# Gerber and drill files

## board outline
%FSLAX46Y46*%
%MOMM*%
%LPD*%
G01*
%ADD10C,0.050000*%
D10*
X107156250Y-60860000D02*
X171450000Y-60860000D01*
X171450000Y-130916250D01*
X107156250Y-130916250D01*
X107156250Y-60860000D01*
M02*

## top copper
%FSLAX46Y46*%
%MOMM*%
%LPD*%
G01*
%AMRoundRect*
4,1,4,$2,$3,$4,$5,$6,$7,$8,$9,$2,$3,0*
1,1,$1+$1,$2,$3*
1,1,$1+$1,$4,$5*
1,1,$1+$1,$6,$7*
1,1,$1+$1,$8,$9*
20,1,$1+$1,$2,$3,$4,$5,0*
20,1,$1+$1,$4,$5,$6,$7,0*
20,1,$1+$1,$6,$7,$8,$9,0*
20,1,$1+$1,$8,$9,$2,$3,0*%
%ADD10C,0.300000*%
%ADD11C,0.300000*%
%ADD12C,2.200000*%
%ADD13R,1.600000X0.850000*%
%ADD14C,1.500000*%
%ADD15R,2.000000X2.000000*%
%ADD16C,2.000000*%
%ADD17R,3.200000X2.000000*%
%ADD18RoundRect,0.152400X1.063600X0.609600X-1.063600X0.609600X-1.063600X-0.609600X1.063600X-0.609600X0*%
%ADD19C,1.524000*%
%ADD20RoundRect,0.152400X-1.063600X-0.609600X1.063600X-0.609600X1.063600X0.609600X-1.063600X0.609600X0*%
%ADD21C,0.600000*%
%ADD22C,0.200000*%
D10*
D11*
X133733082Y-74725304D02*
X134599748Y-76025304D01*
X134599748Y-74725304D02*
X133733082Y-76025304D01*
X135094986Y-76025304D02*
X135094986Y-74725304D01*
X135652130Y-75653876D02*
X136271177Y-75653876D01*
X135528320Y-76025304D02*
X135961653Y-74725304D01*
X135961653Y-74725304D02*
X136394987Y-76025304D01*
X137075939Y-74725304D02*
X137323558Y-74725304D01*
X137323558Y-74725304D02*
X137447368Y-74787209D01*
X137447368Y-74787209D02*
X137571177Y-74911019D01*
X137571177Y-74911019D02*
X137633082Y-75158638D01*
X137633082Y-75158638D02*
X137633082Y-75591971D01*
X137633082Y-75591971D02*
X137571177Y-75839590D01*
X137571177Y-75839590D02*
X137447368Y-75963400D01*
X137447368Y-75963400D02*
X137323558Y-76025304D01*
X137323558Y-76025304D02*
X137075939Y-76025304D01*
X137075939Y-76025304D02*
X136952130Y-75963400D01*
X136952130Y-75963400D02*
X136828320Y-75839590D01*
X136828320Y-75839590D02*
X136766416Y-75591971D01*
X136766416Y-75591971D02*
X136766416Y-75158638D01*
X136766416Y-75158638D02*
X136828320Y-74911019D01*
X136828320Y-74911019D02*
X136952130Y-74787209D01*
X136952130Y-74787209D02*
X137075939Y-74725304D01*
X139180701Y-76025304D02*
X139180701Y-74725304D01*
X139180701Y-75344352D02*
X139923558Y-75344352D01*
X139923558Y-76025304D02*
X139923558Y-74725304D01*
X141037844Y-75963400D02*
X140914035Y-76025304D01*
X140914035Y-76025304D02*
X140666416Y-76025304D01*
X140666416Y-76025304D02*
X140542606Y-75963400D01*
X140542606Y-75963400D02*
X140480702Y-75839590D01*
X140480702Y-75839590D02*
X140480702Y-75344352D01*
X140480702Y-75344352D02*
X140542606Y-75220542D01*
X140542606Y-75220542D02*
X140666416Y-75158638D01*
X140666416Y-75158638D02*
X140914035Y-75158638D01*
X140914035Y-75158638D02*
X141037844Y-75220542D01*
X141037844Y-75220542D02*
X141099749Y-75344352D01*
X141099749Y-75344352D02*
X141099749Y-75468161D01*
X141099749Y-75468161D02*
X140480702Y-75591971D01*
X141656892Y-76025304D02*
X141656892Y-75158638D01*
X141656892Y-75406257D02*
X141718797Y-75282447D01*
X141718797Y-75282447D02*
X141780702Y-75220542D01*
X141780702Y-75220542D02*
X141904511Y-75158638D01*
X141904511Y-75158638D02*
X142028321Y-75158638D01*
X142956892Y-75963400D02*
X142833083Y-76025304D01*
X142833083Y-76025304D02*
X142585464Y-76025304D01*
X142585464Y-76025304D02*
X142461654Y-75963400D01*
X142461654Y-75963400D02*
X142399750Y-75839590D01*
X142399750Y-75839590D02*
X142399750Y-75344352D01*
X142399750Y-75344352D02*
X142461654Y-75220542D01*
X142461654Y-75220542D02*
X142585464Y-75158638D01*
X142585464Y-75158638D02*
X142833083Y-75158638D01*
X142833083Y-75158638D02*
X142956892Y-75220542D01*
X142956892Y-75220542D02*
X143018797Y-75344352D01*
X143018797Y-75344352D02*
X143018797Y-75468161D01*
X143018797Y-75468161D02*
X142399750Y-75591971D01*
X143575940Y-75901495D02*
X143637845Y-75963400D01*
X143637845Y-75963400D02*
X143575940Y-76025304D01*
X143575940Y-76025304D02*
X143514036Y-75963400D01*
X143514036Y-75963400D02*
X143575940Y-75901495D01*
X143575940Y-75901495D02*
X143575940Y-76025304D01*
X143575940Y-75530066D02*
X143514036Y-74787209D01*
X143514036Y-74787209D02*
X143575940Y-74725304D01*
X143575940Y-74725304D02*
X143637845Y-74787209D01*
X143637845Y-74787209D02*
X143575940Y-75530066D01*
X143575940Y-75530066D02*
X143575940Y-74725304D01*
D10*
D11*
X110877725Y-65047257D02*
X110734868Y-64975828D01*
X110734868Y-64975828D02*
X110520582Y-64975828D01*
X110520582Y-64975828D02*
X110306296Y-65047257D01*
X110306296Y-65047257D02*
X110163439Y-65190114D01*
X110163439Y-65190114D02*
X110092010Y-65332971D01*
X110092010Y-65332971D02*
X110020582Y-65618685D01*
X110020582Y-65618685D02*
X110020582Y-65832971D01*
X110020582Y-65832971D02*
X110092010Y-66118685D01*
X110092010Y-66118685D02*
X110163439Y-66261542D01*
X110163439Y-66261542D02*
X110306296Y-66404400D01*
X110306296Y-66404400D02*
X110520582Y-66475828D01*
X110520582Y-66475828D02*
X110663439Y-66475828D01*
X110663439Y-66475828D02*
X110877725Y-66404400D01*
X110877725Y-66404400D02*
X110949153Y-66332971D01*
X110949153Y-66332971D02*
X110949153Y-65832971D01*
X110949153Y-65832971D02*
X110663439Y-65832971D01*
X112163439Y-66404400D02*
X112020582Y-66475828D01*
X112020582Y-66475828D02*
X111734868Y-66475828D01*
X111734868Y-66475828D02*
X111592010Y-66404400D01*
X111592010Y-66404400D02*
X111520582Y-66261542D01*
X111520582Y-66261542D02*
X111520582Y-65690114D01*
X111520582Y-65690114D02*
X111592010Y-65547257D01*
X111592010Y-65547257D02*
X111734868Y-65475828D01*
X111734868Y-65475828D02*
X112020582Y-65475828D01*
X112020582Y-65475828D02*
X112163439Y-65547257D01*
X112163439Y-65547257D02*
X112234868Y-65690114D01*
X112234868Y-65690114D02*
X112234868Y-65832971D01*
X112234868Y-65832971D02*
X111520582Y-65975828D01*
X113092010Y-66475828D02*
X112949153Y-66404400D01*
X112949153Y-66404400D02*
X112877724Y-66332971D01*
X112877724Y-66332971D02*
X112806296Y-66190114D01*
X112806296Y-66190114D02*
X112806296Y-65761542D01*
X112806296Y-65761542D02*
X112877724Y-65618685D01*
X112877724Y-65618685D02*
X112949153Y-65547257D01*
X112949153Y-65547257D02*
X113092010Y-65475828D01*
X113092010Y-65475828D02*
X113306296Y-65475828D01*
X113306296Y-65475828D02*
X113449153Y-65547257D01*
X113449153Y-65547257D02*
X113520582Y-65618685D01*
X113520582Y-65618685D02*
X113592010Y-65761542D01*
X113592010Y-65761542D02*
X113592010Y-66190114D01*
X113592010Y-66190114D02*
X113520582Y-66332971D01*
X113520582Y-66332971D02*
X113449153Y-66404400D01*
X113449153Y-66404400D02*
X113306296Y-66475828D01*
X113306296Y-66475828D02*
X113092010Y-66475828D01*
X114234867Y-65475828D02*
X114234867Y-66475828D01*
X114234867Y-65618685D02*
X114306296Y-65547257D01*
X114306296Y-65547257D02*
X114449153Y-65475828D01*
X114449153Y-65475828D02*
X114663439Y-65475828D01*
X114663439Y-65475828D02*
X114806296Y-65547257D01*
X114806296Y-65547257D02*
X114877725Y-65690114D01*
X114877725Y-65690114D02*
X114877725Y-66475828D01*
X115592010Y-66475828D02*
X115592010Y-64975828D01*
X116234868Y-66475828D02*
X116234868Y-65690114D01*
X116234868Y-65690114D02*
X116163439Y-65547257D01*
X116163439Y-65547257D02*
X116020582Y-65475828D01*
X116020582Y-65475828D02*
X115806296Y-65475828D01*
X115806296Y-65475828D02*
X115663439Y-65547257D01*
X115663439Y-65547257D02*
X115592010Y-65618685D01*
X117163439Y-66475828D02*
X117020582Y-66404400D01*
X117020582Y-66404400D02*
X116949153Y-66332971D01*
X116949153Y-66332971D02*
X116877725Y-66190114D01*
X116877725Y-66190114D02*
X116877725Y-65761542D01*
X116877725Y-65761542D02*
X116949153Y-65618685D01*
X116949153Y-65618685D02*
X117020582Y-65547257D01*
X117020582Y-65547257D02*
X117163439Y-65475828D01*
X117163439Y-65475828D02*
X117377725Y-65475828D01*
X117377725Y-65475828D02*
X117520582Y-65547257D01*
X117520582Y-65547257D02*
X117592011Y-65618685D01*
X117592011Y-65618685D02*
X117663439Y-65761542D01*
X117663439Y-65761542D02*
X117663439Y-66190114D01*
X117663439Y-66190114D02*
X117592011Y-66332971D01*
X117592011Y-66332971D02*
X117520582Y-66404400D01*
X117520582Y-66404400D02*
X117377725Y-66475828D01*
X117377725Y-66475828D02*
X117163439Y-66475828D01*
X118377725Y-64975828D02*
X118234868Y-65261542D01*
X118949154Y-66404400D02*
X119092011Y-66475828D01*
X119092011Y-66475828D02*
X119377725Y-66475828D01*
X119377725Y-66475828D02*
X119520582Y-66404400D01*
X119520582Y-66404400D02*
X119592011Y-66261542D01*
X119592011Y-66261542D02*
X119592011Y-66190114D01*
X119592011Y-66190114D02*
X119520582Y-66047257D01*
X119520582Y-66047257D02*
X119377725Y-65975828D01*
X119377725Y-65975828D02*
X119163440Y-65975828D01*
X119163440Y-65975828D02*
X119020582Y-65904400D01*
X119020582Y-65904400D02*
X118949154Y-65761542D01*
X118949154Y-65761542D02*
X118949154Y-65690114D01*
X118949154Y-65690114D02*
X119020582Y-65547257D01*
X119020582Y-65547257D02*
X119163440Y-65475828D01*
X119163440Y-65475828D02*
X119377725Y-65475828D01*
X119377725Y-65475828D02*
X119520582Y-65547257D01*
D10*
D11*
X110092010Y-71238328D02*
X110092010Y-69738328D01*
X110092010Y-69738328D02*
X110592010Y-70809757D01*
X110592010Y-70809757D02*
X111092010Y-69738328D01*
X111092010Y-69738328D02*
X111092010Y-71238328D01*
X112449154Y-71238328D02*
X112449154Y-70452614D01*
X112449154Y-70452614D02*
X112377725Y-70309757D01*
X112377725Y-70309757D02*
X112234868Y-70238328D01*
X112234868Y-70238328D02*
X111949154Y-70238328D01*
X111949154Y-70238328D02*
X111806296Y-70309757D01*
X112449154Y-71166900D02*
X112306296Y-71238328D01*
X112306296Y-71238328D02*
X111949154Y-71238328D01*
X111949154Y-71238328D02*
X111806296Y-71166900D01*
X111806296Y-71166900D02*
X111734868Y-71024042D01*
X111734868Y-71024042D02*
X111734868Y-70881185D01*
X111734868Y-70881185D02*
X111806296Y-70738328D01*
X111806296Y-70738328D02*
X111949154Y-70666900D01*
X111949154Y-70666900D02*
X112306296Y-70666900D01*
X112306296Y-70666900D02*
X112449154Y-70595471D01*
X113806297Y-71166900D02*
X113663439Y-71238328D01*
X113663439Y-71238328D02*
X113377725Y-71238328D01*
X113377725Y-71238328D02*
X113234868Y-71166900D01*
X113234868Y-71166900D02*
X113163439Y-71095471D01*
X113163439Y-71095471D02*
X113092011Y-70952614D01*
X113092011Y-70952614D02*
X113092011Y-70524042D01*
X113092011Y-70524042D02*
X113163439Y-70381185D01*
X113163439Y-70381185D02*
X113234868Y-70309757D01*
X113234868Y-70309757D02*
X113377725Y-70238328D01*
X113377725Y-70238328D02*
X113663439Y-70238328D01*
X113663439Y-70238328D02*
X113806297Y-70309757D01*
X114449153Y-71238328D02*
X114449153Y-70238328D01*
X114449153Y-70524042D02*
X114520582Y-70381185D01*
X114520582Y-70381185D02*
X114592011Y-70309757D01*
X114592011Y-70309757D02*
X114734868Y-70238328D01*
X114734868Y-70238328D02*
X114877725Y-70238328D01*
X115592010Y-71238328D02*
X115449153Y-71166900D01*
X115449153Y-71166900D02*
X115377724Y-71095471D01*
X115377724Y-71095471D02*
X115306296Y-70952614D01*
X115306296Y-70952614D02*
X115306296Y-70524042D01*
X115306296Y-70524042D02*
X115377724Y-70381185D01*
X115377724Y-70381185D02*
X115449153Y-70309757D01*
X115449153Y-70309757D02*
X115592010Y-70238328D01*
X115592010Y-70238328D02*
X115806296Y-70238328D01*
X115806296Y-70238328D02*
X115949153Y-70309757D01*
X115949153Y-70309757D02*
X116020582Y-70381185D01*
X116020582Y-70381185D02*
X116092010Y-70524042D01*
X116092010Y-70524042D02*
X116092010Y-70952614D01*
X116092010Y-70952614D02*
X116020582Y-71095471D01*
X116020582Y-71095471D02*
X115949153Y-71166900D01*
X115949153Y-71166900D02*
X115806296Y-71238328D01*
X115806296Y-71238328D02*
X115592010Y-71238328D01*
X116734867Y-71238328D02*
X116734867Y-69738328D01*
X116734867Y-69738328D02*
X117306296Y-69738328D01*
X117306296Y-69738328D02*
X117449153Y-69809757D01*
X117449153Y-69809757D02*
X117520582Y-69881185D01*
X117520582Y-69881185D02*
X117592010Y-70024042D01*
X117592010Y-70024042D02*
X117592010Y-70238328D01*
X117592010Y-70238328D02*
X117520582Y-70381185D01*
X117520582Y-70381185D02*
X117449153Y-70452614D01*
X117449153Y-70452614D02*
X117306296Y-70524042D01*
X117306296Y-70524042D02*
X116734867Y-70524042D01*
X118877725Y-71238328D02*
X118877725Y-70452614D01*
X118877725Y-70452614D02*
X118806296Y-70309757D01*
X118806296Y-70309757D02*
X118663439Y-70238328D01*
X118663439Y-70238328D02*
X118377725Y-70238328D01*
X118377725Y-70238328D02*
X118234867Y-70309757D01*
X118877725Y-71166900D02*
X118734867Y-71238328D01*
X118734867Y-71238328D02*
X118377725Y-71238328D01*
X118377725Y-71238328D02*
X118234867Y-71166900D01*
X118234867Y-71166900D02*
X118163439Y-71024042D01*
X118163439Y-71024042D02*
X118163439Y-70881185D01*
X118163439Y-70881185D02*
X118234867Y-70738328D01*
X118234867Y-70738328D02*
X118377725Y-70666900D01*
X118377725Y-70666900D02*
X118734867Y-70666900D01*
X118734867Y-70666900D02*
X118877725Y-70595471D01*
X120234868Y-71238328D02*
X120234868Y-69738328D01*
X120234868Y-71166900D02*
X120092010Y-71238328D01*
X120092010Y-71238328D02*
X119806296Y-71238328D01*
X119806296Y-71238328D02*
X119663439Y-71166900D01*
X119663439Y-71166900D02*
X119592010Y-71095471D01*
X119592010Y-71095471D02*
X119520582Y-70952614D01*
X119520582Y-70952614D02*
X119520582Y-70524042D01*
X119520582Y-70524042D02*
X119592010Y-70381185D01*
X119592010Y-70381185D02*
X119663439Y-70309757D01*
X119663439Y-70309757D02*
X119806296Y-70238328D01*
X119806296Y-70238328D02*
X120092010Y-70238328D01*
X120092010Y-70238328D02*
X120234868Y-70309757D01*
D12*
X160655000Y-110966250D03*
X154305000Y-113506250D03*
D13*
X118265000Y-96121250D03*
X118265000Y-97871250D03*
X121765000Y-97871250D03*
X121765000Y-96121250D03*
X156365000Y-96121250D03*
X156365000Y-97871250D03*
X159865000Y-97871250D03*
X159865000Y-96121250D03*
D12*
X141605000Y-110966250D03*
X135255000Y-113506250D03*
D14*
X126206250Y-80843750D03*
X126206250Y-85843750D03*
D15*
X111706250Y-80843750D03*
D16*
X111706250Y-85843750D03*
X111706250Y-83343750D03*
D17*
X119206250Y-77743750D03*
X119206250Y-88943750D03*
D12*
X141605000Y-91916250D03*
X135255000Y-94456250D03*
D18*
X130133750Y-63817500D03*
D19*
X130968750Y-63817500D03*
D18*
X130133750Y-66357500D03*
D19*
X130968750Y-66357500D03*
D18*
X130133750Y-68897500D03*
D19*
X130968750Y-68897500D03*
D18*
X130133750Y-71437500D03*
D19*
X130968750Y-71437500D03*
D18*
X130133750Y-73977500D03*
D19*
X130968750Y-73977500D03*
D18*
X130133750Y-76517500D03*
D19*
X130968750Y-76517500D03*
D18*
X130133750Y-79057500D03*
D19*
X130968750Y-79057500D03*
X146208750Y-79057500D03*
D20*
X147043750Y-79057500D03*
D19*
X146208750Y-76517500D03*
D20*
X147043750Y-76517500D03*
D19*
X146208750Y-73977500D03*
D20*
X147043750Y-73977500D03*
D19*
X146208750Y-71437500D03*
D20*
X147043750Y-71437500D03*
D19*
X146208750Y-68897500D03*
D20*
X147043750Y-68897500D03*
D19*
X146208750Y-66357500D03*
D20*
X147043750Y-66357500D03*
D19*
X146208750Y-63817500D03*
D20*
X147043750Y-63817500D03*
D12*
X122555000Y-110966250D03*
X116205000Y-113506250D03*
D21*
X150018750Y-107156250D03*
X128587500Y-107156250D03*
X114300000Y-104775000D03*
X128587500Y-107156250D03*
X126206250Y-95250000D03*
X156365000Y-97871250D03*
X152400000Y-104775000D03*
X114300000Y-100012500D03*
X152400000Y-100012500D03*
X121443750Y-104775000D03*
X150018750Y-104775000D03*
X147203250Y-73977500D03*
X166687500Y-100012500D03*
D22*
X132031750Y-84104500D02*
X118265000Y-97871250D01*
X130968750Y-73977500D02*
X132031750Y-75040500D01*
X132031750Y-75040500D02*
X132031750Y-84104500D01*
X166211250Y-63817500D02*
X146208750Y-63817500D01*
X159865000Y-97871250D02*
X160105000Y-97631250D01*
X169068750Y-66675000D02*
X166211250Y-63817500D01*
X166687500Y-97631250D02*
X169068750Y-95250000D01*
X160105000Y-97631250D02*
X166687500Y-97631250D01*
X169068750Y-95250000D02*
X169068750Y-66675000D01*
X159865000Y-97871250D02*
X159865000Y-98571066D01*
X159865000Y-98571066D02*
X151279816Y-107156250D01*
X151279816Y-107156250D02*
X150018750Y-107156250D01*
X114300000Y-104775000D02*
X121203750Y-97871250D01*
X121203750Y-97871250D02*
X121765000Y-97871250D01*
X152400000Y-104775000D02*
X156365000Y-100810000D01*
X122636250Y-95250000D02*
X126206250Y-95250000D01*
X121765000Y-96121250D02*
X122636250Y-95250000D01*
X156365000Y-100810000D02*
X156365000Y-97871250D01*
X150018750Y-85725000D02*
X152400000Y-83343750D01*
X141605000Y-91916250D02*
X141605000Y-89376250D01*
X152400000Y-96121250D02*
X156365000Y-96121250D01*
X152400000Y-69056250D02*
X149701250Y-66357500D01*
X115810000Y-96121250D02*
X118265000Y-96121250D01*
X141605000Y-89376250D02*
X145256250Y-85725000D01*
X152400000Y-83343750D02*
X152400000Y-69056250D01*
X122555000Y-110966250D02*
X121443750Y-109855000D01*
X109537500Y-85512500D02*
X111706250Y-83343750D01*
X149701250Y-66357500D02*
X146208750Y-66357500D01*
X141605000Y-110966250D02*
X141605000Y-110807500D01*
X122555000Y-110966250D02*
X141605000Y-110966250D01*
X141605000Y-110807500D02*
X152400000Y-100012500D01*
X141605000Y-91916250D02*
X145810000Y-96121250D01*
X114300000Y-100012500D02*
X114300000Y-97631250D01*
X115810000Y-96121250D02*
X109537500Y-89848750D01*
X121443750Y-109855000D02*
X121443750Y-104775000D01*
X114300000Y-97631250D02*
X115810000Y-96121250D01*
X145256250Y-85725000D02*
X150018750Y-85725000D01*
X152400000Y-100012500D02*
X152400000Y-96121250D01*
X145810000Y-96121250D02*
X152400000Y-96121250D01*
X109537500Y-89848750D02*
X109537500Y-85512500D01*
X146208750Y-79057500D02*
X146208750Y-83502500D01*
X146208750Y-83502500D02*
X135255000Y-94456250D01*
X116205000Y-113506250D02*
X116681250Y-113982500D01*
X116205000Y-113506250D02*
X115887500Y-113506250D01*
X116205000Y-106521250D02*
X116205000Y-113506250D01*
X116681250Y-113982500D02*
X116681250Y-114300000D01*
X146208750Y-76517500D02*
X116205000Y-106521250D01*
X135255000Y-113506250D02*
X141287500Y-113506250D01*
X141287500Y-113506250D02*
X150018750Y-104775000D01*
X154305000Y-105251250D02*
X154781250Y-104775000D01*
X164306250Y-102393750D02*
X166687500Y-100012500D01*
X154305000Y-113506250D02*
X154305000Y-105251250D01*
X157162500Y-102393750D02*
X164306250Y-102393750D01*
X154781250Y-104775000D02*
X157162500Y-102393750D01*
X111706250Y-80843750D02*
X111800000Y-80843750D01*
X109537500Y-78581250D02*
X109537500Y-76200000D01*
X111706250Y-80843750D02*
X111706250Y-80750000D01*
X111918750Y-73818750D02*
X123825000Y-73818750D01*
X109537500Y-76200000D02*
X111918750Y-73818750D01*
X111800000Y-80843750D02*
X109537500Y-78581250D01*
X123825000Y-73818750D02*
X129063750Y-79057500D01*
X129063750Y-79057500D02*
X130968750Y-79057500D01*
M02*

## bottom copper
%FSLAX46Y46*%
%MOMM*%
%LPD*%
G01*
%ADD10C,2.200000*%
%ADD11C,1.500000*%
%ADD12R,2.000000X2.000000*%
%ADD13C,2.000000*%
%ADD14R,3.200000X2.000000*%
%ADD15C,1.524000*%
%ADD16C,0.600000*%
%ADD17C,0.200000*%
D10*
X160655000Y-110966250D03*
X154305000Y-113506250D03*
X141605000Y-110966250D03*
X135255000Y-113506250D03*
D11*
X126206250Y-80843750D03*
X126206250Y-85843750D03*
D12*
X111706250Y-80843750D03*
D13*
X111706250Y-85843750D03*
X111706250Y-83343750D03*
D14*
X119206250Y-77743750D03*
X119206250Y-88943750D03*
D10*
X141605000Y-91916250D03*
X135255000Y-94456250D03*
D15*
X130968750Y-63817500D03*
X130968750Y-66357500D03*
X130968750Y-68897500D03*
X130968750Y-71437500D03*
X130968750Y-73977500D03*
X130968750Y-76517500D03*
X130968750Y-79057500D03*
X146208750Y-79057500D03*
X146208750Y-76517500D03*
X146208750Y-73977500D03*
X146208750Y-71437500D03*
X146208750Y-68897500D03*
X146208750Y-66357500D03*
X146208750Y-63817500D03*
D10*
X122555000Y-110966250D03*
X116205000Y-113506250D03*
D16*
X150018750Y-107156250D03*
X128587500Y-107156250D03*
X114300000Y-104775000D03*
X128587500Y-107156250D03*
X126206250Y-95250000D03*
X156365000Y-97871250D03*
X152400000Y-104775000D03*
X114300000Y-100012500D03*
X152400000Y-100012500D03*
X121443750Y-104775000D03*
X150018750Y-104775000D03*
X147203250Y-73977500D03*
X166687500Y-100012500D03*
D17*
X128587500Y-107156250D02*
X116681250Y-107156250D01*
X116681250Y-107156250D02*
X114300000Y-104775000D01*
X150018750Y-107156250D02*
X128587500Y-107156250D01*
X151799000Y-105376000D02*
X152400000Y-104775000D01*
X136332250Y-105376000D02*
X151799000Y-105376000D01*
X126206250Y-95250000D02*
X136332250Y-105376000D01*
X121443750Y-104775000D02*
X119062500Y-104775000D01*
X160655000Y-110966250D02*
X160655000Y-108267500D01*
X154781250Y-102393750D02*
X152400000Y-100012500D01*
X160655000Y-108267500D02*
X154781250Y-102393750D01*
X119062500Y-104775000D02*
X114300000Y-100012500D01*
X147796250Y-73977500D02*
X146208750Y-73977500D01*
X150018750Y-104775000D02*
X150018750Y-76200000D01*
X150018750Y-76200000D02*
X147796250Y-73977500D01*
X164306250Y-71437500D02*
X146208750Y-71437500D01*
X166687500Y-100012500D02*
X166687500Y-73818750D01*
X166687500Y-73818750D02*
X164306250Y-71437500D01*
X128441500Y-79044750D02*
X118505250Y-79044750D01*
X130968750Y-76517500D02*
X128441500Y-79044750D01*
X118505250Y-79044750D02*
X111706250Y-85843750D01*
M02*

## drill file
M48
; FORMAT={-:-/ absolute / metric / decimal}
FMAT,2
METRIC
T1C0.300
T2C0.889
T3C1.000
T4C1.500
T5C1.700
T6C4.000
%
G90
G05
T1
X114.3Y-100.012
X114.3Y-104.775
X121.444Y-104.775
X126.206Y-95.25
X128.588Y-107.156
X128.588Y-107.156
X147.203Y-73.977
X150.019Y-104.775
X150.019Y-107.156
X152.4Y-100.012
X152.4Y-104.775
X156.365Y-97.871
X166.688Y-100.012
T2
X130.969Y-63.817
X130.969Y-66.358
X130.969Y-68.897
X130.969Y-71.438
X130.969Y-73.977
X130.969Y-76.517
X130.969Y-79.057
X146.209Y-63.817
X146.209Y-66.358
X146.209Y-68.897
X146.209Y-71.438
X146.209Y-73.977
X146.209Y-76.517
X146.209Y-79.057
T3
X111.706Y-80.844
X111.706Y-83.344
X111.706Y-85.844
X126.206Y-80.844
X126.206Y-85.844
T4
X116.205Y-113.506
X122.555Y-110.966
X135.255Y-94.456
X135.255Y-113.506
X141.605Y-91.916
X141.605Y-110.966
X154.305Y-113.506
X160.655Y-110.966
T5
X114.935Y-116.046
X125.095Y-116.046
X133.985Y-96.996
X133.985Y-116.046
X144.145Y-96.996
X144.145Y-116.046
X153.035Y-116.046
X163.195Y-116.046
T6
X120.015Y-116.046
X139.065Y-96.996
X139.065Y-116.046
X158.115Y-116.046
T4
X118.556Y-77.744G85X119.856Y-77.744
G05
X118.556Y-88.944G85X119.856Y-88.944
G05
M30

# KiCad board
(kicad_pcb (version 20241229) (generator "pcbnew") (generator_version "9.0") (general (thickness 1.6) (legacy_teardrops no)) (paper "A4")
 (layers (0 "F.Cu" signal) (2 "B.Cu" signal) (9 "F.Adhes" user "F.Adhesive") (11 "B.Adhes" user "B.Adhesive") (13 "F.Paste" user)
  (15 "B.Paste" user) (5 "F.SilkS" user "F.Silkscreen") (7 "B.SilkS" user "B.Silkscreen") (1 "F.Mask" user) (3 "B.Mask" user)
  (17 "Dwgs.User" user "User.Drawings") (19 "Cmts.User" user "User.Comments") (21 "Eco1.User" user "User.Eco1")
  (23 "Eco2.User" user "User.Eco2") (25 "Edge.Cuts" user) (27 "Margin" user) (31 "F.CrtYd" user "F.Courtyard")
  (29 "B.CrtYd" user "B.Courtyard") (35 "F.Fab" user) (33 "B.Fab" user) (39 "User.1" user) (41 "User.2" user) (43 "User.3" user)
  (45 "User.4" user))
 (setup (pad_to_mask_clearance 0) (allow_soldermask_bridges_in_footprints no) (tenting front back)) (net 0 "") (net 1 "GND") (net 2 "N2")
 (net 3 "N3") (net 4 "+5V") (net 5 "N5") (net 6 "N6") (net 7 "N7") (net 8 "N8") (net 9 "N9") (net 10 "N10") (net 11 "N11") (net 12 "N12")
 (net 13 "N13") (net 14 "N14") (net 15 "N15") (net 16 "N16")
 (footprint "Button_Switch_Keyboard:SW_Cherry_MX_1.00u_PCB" (layer "F.Cu") (at 160.655 110.96625)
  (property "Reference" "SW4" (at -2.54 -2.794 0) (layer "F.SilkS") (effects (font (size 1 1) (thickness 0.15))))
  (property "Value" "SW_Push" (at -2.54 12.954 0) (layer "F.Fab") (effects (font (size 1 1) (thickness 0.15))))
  (pad "" np_thru_hole circle (at -7.62 5.08) (size 1.7 1.7) (drill 1.7) (layers "*.Cu" "*.Mask"))
  (pad "" np_thru_hole circle (at -2.54 5.08) (size 4 4) (drill 4) (layers "*.Cu" "*.Mask"))
  (pad "" np_thru_hole circle (at 2.54 5.08) (size 1.7 1.7) (drill 1.7) (layers "*.Cu" "*.Mask"))
  (pad "1" thru_hole circle (at 0 0) (size 2.2 2.2) (drill 1.5) (layers "*.Cu" "*.Mask") (remove_unused_layers no) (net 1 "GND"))
  (pad "2" thru_hole circle (at -6.35 2.54) (size 2.2 2.2) (drill 1.5) (layers "*.Cu" "*.Mask") (remove_unused_layers no) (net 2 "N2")))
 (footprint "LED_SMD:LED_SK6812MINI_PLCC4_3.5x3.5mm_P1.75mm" (layer "F.Cu") (at 120.015 96.99625)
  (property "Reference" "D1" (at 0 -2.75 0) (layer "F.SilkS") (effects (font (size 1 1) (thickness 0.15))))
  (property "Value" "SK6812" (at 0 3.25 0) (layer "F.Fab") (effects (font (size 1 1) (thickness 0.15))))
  (pad "1" smd rect (at -1.75 -0.875) (size 1.6 0.85) (layers "F.Cu" "F.Mask" "F.Paste") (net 1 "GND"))
  (pad "2" smd rect (at -1.75 0.875) (size 1.6 0.85) (layers "F.Cu" "F.Mask" "F.Paste") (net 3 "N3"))
  (pad "3" smd rect (at 1.75 0.875) (size 1.6 0.85) (layers "F.Cu" "F.Mask" "F.Paste") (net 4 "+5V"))
  (pad "4" smd rect (at 1.75 -0.875) (size 1.6 0.85) (layers "F.Cu" "F.Mask" "F.Paste") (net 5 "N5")))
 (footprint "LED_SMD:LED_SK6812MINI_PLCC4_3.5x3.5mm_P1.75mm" (layer "F.Cu") (at 158.115 96.99625)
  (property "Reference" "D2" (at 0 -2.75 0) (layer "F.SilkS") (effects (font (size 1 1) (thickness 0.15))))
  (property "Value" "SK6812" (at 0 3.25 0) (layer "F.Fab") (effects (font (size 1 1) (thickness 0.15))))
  (pad "1" smd rect (at -1.75 -0.875) (size 1.6 0.85) (layers "F.Cu" "F.Mask" "F.Paste") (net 1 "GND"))
  (pad "2" smd rect (at -1.75 0.875) (size 1.6 0.85) (layers "F.Cu" "F.Mask" "F.Paste") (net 5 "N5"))
  (pad "3" smd rect (at 1.75 0.875) (size 1.6 0.85) (layers "F.Cu" "F.Mask" "F.Paste") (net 4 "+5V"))
  (pad "4" smd rect (at 1.75 -0.875) (size 1.6 0.85) (layers "F.Cu" "F.Mask" "F.Paste") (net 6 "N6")))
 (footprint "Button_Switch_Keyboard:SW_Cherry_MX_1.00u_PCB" (layer "F.Cu") (at 141.605 110.96625)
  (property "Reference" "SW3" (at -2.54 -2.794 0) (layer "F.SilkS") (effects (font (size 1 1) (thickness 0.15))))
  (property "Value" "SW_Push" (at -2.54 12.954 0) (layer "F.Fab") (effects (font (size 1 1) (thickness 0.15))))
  (pad "" np_thru_hole circle (at -7.62 5.08) (size 1.7 1.7) (drill 1.7) (layers "*.Cu" "*.Mask"))
  (pad "" np_thru_hole circle (at -2.54 5.08) (size 4 4) (drill 4) (layers "*.Cu" "*.Mask"))
  (pad "" np_thru_hole circle (at 2.54 5.08) (size 1.7 1.7) (drill 1.7) (layers "*.Cu" "*.Mask"))
  (pad "1" thru_hole circle (at 0 0) (size 2.2 2.2) (drill 1.5) (layers "*.Cu" "*.Mask") (remove_unused_layers no) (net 1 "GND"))
  (pad "2" thru_hole circle (at -6.35 2.54) (size 2.2 2.2) (drill 1.5) (layers "*.Cu" "*.Mask") (remove_unused_layers no) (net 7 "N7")))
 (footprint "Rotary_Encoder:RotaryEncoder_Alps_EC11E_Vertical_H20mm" (layer "F.Cu") (at 111.70625 80.84375)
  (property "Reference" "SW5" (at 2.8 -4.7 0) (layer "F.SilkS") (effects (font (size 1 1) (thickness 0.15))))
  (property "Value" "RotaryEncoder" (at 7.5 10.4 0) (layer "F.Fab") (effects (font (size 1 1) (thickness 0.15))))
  (pad "" thru_hole circle (at 14.5 0) (size 1.5 1.5) (drill 1) (layers "*.Cu" "*.Mask") (remove_unused_layers no))
  (pad "" thru_hole circle (at 14.5 5) (size 1.5 1.5) (drill 1) (layers "*.Cu" "*.Mask") (remove_unused_layers no))
  (pad "A" thru_hole rect (at 0 0) (size 2 2) (drill 1) (layers "*.Cu" "*.Mask") (remove_unused_layers no) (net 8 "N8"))
  (pad "B" thru_hole circle (at 0 5) (size 2 2) (drill 1) (layers "*.Cu" "*.Mask") (remove_unused_layers no) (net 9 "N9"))
  (pad "C" thru_hole circle (at 0 2.5) (size 2 2) (drill 1) (layers "*.Cu" "*.Mask") (remove_unused_layers no) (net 1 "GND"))
  (pad "MP" thru_hole rect (at 7.5 -3.1) (size 3.2 2) (drill oval 2.8 1.5) (layers "*.Cu" "*.Mask") (remove_unused_layers no))
  (pad "MP" thru_hole rect (at 7.5 8.1) (size 3.2 2) (drill oval 2.8 1.5) (layers "*.Cu" "*.Mask") (remove_unused_layers no)))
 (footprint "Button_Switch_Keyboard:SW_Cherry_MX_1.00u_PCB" (layer "F.Cu") (at 141.605 91.91625)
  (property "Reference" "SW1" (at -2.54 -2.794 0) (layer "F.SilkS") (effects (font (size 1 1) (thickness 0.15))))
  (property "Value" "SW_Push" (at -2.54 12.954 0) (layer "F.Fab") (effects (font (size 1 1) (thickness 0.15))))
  (pad "" np_thru_hole circle (at -7.62 5.08) (size 1.7 1.7) (drill 1.7) (layers "*.Cu" "*.Mask"))
  (pad "" np_thru_hole circle (at -2.54 5.08) (size 4 4) (drill 4) (layers "*.Cu" "*.Mask"))
  (pad "" np_thru_hole circle (at 2.54 5.08) (size 1.7 1.7) (drill 1.7) (layers "*.Cu" "*.Mask"))
  (pad "1" thru_hole circle (at 0 0) (size 2.2 2.2) (drill 1.5) (layers "*.Cu" "*.Mask") (remove_unused_layers no) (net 1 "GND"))
  (pad "2" thru_hole circle (at -6.35 2.54) (size 2.2 2.2) (drill 1.5) (layers "*.Cu" "*.Mask") (remove_unused_layers no) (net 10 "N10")))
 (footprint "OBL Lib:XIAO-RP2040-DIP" (layer "F.Cu") (at 138.58875 71.4375)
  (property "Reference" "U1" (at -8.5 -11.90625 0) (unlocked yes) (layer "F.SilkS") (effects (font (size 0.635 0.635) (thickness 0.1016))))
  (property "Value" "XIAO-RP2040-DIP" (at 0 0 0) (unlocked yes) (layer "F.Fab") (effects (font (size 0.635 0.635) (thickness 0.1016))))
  (pad "1" smd roundrect (at -8.455 -7.62 180) (size 2.432 1.524) (layers "F.Cu" "F.Mask") (roundrect_rratio 0.1) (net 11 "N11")
   (thermal_bridge_angle 45))
  (pad "1" thru_hole circle (at -7.62 -7.62 180) (size 1.524 1.524) (drill 0.889) (layers "*.Cu" "*.Mask") (remove_unused_layers no)
   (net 11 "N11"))
  (pad "2" smd roundrect (at -8.455 -5.08 180) (size 2.432 1.524) (layers "F.Cu" "F.Mask") (roundrect_rratio 0.1) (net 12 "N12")
   (thermal_bridge_angle 45))
  (pad "2" thru_hole circle (at -7.62 -5.08 180) (size 1.524 1.524) (drill 0.889) (layers "*.Cu" "*.Mask") (remove_unused_layers no)
   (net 12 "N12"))
  (pad "3" smd roundrect (at -8.455 -2.54 180) (size 2.432 1.524) (layers "F.Cu" "F.Mask") (roundrect_rratio 0.1) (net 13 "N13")
   (thermal_bridge_angle 45))
  (pad "3" thru_hole circle (at -7.62 -2.54 180) (size 1.524 1.524) (drill 0.889) (layers "*.Cu" "*.Mask") (remove_unused_layers no)
   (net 13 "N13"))
  (pad "4" smd roundrect (at -8.455 0 180) (size 2.432 1.524) (layers "F.Cu" "F.Mask") (roundrect_rratio 0.1) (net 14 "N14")
   (thermal_bridge_angle 45))
  (pad "4" thru_hole circle (at -7.62 0 180) (size 1.524 1.524) (drill 0.889) (layers "*.Cu" "*.Mask") (remove_unused_layers no)
   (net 14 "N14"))
  (pad "5" smd roundrect (at -8.455 2.54 180) (size 2.432 1.524) (layers "F.Cu" "F.Mask") (roundrect_rratio 0.1) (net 3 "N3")
   (thermal_bridge_angle 45))
  (pad "5" thru_hole circle (at -7.62 2.54 180) (size 1.524 1.524) (drill 0.889) (layers "*.Cu" "*.Mask") (remove_unused_layers no)
   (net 3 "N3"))
  (pad "6" smd roundrect (at -8.455 5.08 180) (size 2.432 1.524) (layers "F.Cu" "F.Mask") (roundrect_rratio 0.1) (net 9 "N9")
   (thermal_bridge_angle 45))
  (pad "6" thru_hole circle (at -7.62 5.08 180) (size 1.524 1.524) (drill 0.889) (layers "*.Cu" "*.Mask") (remove_unused_layers no)
   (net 9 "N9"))
  (pad "7" smd roundrect (at -8.455 7.62 180) (size 2.432 1.524) (layers "F.Cu" "F.Mask") (roundrect_rratio 0.1) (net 8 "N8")
   (thermal_bridge_angle 45))
  (pad "7" thru_hole circle (at -7.62 7.62 180) (size 1.524 1.524) (drill 0.889) (layers "*.Cu" "*.Mask") (remove_unused_layers no)
   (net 8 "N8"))
  (pad "8" thru_hole circle (at 7.62 7.62) (size 1.524 1.524) (drill 0.889) (layers "*.Cu" "*.Mask") (remove_unused_layers no)
   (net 10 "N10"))
  (pad "8" smd roundrect (at 8.455 7.62) (size 2.432 1.524) (layers "F.Cu" "F.Mask") (roundrect_rratio 0.1) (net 10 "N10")
   (thermal_bridge_angle 45))
  (pad "9" thru_hole circle (at 7.62 5.08) (size 1.524 1.524) (drill 0.889) (layers "*.Cu" "*.Mask") (remove_unused_layers no)
   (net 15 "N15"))
  (pad "9" smd roundrect (at 8.455 5.08) (size 2.432 1.524) (layers "F.Cu" "F.Mask") (roundrect_rratio 0.1) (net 15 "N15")
   (thermal_bridge_angle 45))
  (pad "10" thru_hole circle (at 7.62 2.54) (size 1.524 1.524) (drill 0.889) (layers "*.Cu" "*.Mask") (remove_unused_layers no) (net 7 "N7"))
  (pad "10" smd roundrect (at 8.455 2.54) (size 2.432 1.524) (layers "F.Cu" "F.Mask") (roundrect_rratio 0.1) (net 7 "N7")
   (thermal_bridge_angle 45))
  (pad "11" thru_hole circle (at 7.62 0) (size 1.524 1.524) (drill 0.889) (layers "*.Cu" "*.Mask") (remove_unused_layers no) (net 2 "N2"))
  (pad "11" smd roundrect (at 8.455 0) (size 2.432 1.524) (layers "F.Cu" "F.Mask") (roundrect_rratio 0.1) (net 2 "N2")
   (thermal_bridge_angle 45))
  (pad "12" thru_hole circle (at 7.62 -2.54) (size 1.524 1.524) (drill 0.889) (layers "*.Cu" "*.Mask") (remove_unused_layers no)
   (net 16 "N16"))
  (pad "12" smd roundrect (at 8.455 -2.54) (size 2.432 1.524) (layers "F.Cu" "F.Mask") (roundrect_rratio 0.1) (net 16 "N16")
   (thermal_bridge_angle 45))
  (pad "13" thru_hole circle (at 7.62 -5.08) (size 1.524 1.524) (drill 0.889) (layers "*.Cu" "*.Mask") (remove_unused_layers no)
   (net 1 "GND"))
  (pad "13" smd roundrect (at 8.455 -5.08) (size 2.432 1.524) (layers "F.Cu" "F.Mask") (roundrect_rratio 0.1) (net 1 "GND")
   (thermal_bridge_angle 45))
  (pad "14" thru_hole circle (at 7.62 -7.62) (size 1.524 1.524) (drill 0.889) (layers "*.Cu" "*.Mask") (remove_unused_layers no)
   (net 4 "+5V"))
  (pad "14" smd roundrect (at 8.455 -7.62) (size 2.432 1.524) (layers "F.Cu" "F.Mask") (roundrect_rratio 0.1) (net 4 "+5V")
   (thermal_bridge_angle 45)))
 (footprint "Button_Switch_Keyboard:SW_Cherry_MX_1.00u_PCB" (layer "F.Cu") (at 122.555 110.96625)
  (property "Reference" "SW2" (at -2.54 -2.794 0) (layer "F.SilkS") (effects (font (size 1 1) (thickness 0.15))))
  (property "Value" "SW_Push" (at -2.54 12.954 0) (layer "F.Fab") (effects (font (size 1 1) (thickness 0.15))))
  (pad "" np_thru_hole circle (at -7.62 5.08) (size 1.7 1.7) (drill 1.7) (layers "*.Cu" "*.Mask"))
  (pad "" np_thru_hole circle (at -2.54 5.08) (size 4 4) (drill 4) (layers "*.Cu" "*.Mask"))
  (pad "" np_thru_hole circle (at 2.54 5.08) (size 1.7 1.7) (drill 1.7) (layers "*.Cu" "*.Mask"))
  (pad "1" thru_hole circle (at 0 0) (size 2.2 2.2) (drill 1.5) (layers "*.Cu" "*.Mask") (remove_unused_layers no) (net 1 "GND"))
  (pad "2" thru_hole circle (at -6.35 2.54) (size 2.2 2.2) (drill 1.5) (layers "*.Cu" "*.Mask") (remove_unused_layers no) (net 15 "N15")))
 (gr_rect (start 107.15625 60.86) (end 171.45 130.91625) (stroke (width 0.05) (type default)) (fill no) (layer "Edge.Cuts"))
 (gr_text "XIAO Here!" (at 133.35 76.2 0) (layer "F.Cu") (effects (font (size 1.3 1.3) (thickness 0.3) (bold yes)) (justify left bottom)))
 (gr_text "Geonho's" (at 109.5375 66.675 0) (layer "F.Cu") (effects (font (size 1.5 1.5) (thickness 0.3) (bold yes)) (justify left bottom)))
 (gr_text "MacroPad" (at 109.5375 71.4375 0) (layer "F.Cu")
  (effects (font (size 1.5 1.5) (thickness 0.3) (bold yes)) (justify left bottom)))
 (segment (start 132.03175 84.1045) (end 118.265 97.87125) (width 0.2) (layer "F.Cu") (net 3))
 (segment (start 130.96875 73.9775) (end 132.03175 75.0405) (width 0.2) (layer "F.Cu") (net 3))
 (segment (start 132.03175 75.0405) (end 132.03175 84.1045) (width 0.2) (layer "F.Cu") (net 3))
 (segment (start 166.21125 63.8175) (end 146.20875 63.8175) (width 0.2) (layer "F.Cu") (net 4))
 (segment (start 159.865 97.87125) (end 160.105 97.63125) (width 0.2) (layer "F.Cu") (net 4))
 (segment (start 169.06875 66.675) (end 166.21125 63.8175) (width 0.2) (layer "F.Cu") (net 4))
 (segment (start 166.6875 97.63125) (end 169.06875 95.25) (width 0.2) (layer "F.Cu") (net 4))
 (segment (start 160.105 97.63125) (end 166.6875 97.63125) (width 0.2) (layer "F.Cu") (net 4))
 (segment (start 169.06875 95.25) (end 169.06875 66.675) (width 0.2) (layer "F.Cu") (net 4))
 (segment (start 159.865 97.87125) (end 159.865 98.571066) (width 0.2) (layer "F.Cu") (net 4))
 (segment (start 159.865 98.571066) (end 151.279816 107.15625) (width 0.2) (layer "F.Cu") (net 4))
 (segment (start 151.279816 107.15625) (end 150.01875 107.15625) (width 0.2) (layer "F.Cu") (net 4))
 (segment (start 114.3 104.775) (end 121.20375 97.87125) (width 0.2) (layer "F.Cu") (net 4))
 (segment (start 121.20375 97.87125) (end 121.765 97.87125) (width 0.2) (layer "F.Cu") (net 4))
 (via (at 150.01875 107.15625) (size 0.6) (drill 0.3) (layers "F.Cu" "B.Cu") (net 4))
 (via (at 128.5875 107.15625) (size 0.6) (drill 0.3) (layers "F.Cu" "B.Cu") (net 4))
 (via (at 114.3 104.775) (size 0.6) (drill 0.3) (layers "F.Cu" "B.Cu") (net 4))
 (via (at 128.5875 107.15625) (size 0.6) (drill 0.3) (layers "F.Cu" "B.Cu") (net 4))
 (segment (start 128.5875 107.15625) (end 116.68125 107.15625) (width 0.2) (layer "B.Cu") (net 4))
 (segment (start 116.68125 107.15625) (end 114.3 104.775) (width 0.2) (layer "B.Cu") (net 4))
 (segment (start 150.01875 107.15625) (end 128.5875 107.15625) (width 0.2) (layer "B.Cu") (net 4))
 (segment (start 152.4 104.775) (end 156.365 100.81) (width 0.2) (layer "F.Cu") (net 5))
 (segment (start 122.63625 95.25) (end 126.20625 95.25) (width 0.2) (layer "F.Cu") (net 5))
 (segment (start 121.765 96.12125) (end 122.63625 95.25) (width 0.2) (layer "F.Cu") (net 5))
 (segment (start 156.365 100.81) (end 156.365 97.87125) (width 0.2) (layer "F.Cu") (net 5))
 (via (at 126.20625 95.25) (size 0.6) (drill 0.3) (layers "F.Cu" "B.Cu") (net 5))
 (via (at 156.365 97.87125) (size 0.6) (drill 0.3) (layers "F.Cu" "B.Cu") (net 5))
 (via (at 152.4 104.775) (size 0.6) (drill 0.3) (layers "F.Cu" "B.Cu") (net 5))
 (segment (start 151.799 105.376) (end 152.4 104.775) (width 0.2) (layer "B.Cu") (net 5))
 (segment (start 136.33225 105.376) (end 151.799 105.376) (width 0.2) (layer "B.Cu") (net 5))
 (segment (start 126.20625 95.25) (end 136.33225 105.376) (width 0.2) (layer "B.Cu") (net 5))
 (segment (start 150.01875 85.725) (end 152.4 83.34375) (width 0.2) (layer "F.Cu") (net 1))
 (segment (start 141.605 91.91625) (end 141.605 89.37625) (width 0.2) (layer "F.Cu") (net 1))
 (segment (start 152.4 96.12125) (end 156.365 96.12125) (width 0.2) (layer "F.Cu") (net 1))
 (segment (start 152.4 69.05625) (end 149.70125 66.3575) (width 0.2) (layer "F.Cu") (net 1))
 (segment (start 115.81 96.12125) (end 118.265 96.12125) (width 0.2) (layer "F.Cu") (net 1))
 (segment (start 141.605 89.37625) (end 145.25625 85.725) (width 0.2) (layer "F.Cu") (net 1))
 (segment (start 152.4 83.34375) (end 152.4 69.05625) (width 0.2) (layer "F.Cu") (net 1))
 (segment (start 122.555 110.96625) (end 121.44375 109.855) (width 0.2) (layer "F.Cu") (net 1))
 (segment (start 109.5375 85.5125) (end 111.70625 83.34375) (width 0.2) (layer "F.Cu") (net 1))
 (segment (start 149.70125 66.3575) (end 146.20875 66.3575) (width 0.2) (layer "F.Cu") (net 1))
 (segment (start 141.605 110.96625) (end 141.605 110.8075) (width 0.2) (layer "F.Cu") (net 1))
 (segment (start 122.555 110.96625) (end 141.605 110.96625) (width 0.2) (layer "F.Cu") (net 1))
 (segment (start 141.605 110.8075) (end 152.4 100.0125) (width 0.2) (layer "F.Cu") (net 1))
 (segment (start 141.605 91.91625) (end 145.81 96.12125) (width 0.2) (layer "F.Cu") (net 1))
 (segment (start 114.3 100.0125) (end 114.3 97.63125) (width 0.2) (layer "F.Cu") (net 1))
 (segment (start 115.81 96.12125) (end 109.5375 89.84875) (width 0.2) (layer "F.Cu") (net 1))
 (segment (start 121.44375 109.855) (end 121.44375 104.775) (width 0.2) (layer "F.Cu") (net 1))
 (segment (start 114.3 97.63125) (end 115.81 96.12125) (width 0.2) (layer "F.Cu") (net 1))
 (segment (start 145.25625 85.725) (end 150.01875 85.725) (width 0.2) (layer "F.Cu") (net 1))
 (segment (start 152.4 100.0125) (end 152.4 96.12125) (width 0.2) (layer "F.Cu") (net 1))
 (segment (start 145.81 96.12125) (end 152.4 96.12125) (width 0.2) (layer "F.Cu") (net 1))
 (segment (start 109.5375 89.84875) (end 109.5375 85.5125) (width 0.2) (layer "F.Cu") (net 1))
 (via (at 114.3 100.0125) (size 0.6) (drill 0.3) (layers "F.Cu" "B.Cu") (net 1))
 (via (at 152.4 100.0125) (size 0.6) (drill 0.3) (layers "F.Cu" "B.Cu") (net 1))
 (via (at 121.44375 104.775) (size 0.6) (drill 0.3) (layers "F.Cu" "B.Cu") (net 1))
 (segment (start 121.44375 104.775) (end 119.0625 104.775) (width 0.2) (layer "B.Cu") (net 1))
 (segment (start 160.655 110.96625) (end 160.655 108.2675) (width 0.2) (layer "B.Cu") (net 1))
 (segment (start 154.78125 102.39375) (end 152.4 100.0125) (width 0.2) (layer "B.Cu") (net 1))
 (segment (start 160.655 108.2675) (end 154.78125 102.39375) (width 0.2) (layer "B.Cu") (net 1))
 (segment (start 119.0625 104.775) (end 114.3 100.0125) (width 0.2) (layer "B.Cu") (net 1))
 (segment (start 146.20875 79.0575) (end 146.20875 83.5025) (width 0.2) (layer "F.Cu") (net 10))
 (segment (start 146.20875 83.5025) (end 135.255 94.45625) (width 0.2) (layer "F.Cu") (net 10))
 (segment (start 116.205 113.50625) (end 116.68125 113.9825) (width 0.2) (layer "F.Cu") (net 15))
 (segment (start 116.205 113.50625) (end 115.8875 113.50625) (width 0.2) (layer "F.Cu") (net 15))
 (segment (start 116.205 106.52125) (end 116.205 113.50625) (width 0.2) (layer "F.Cu") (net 15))
 (segment (start 116.68125 113.9825) (end 116.68125 114.3) (width 0.2) (layer "F.Cu") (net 15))
 (segment (start 146.20875 76.5175) (end 116.205 106.52125) (width 0.2) (layer "F.Cu") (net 15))
 (segment (start 135.255 113.50625) (end 141.2875 113.50625) (width 0.2) (layer "F.Cu") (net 7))
 (segment (start 141.2875 113.50625) (end 150.01875 104.775) (width 0.2) (layer "F.Cu") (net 7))
 (via (at 150.01875 104.775) (size 0.6) (drill 0.3) (layers "F.Cu" "B.Cu") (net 7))
 (via (at 147.20325 73.9775) (size 0.6) (drill 0.3) (layers "F.Cu" "B.Cu") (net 7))
 (segment (start 147.79625 73.9775) (end 146.20875 73.9775) (width 0.2) (layer "B.Cu") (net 7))
 (segment (start 150.01875 104.775) (end 150.01875 76.2) (width 0.2) (layer "B.Cu") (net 7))
 (segment (start 150.01875 76.2) (end 147.79625 73.9775) (width 0.2) (layer "B.Cu") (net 7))
 (segment (start 154.305 105.25125) (end 154.78125 104.775) (width 0.2) (layer "F.Cu") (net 2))
 (segment (start 164.30625 102.39375) (end 166.6875 100.0125) (width 0.2) (layer "F.Cu") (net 2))
 (segment (start 154.305 113.50625) (end 154.305 105.25125) (width 0.2) (layer "F.Cu") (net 2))
 (segment (start 157.1625 102.39375) (end 164.30625 102.39375) (width 0.2) (layer "F.Cu") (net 2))
 (segment (start 154.78125 104.775) (end 157.1625 102.39375) (width 0.2) (layer "F.Cu") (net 2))
 (via (at 166.6875 100.0125) (size 0.6) (drill 0.3) (layers "F.Cu" "B.Cu") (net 2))
 (segment (start 164.30625 71.4375) (end 146.20875 71.4375) (width 0.2) (layer "B.Cu") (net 2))
 (segment (start 166.6875 100.0125) (end 166.6875 73.81875) (width 0.2) (layer "B.Cu") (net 2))
 (segment (start 166.6875 73.81875) (end 164.30625 71.4375) (width 0.2) (layer "B.Cu") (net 2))
 (segment (start 128.4415 79.04475) (end 118.50525 79.04475) (width 0.2) (layer "B.Cu") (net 9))
 (segment (start 130.96875 76.5175) (end 128.4415 79.04475) (width 0.2) (layer "B.Cu") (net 9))
 (segment (start 118.50525 79.04475) (end 111.70625 85.84375) (width 0.2) (layer "B.Cu") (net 9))
 (segment (start 111.70625 80.84375) (end 111.8 80.84375) (width 0.2) (layer "F.Cu") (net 8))
 (segment (start 109.5375 78.58125) (end 109.5375 76.2) (width 0.2) (layer "F.Cu") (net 8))
 (segment (start 111.70625 80.84375) (end 111.70625 80.75) (width 0.2) (layer "F.Cu") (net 8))
 (segment (start 111.91875 73.81875) (end 123.825 73.81875) (width 0.2) (layer "F.Cu") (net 8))
 (segment (start 109.5375 76.2) (end 111.91875 73.81875) (width 0.2) (layer "F.Cu") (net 8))
 (segment (start 111.8 80.84375) (end 109.5375 78.58125) (width 0.2) (layer "F.Cu") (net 8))
 (segment (start 123.825 73.81875) (end 129.06375 79.0575) (width 0.2) (layer "F.Cu") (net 8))
 (segment (start 129.06375 79.0575) (end 130.96875 79.0575) (width 0.2) (layer "F.Cu") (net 8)))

